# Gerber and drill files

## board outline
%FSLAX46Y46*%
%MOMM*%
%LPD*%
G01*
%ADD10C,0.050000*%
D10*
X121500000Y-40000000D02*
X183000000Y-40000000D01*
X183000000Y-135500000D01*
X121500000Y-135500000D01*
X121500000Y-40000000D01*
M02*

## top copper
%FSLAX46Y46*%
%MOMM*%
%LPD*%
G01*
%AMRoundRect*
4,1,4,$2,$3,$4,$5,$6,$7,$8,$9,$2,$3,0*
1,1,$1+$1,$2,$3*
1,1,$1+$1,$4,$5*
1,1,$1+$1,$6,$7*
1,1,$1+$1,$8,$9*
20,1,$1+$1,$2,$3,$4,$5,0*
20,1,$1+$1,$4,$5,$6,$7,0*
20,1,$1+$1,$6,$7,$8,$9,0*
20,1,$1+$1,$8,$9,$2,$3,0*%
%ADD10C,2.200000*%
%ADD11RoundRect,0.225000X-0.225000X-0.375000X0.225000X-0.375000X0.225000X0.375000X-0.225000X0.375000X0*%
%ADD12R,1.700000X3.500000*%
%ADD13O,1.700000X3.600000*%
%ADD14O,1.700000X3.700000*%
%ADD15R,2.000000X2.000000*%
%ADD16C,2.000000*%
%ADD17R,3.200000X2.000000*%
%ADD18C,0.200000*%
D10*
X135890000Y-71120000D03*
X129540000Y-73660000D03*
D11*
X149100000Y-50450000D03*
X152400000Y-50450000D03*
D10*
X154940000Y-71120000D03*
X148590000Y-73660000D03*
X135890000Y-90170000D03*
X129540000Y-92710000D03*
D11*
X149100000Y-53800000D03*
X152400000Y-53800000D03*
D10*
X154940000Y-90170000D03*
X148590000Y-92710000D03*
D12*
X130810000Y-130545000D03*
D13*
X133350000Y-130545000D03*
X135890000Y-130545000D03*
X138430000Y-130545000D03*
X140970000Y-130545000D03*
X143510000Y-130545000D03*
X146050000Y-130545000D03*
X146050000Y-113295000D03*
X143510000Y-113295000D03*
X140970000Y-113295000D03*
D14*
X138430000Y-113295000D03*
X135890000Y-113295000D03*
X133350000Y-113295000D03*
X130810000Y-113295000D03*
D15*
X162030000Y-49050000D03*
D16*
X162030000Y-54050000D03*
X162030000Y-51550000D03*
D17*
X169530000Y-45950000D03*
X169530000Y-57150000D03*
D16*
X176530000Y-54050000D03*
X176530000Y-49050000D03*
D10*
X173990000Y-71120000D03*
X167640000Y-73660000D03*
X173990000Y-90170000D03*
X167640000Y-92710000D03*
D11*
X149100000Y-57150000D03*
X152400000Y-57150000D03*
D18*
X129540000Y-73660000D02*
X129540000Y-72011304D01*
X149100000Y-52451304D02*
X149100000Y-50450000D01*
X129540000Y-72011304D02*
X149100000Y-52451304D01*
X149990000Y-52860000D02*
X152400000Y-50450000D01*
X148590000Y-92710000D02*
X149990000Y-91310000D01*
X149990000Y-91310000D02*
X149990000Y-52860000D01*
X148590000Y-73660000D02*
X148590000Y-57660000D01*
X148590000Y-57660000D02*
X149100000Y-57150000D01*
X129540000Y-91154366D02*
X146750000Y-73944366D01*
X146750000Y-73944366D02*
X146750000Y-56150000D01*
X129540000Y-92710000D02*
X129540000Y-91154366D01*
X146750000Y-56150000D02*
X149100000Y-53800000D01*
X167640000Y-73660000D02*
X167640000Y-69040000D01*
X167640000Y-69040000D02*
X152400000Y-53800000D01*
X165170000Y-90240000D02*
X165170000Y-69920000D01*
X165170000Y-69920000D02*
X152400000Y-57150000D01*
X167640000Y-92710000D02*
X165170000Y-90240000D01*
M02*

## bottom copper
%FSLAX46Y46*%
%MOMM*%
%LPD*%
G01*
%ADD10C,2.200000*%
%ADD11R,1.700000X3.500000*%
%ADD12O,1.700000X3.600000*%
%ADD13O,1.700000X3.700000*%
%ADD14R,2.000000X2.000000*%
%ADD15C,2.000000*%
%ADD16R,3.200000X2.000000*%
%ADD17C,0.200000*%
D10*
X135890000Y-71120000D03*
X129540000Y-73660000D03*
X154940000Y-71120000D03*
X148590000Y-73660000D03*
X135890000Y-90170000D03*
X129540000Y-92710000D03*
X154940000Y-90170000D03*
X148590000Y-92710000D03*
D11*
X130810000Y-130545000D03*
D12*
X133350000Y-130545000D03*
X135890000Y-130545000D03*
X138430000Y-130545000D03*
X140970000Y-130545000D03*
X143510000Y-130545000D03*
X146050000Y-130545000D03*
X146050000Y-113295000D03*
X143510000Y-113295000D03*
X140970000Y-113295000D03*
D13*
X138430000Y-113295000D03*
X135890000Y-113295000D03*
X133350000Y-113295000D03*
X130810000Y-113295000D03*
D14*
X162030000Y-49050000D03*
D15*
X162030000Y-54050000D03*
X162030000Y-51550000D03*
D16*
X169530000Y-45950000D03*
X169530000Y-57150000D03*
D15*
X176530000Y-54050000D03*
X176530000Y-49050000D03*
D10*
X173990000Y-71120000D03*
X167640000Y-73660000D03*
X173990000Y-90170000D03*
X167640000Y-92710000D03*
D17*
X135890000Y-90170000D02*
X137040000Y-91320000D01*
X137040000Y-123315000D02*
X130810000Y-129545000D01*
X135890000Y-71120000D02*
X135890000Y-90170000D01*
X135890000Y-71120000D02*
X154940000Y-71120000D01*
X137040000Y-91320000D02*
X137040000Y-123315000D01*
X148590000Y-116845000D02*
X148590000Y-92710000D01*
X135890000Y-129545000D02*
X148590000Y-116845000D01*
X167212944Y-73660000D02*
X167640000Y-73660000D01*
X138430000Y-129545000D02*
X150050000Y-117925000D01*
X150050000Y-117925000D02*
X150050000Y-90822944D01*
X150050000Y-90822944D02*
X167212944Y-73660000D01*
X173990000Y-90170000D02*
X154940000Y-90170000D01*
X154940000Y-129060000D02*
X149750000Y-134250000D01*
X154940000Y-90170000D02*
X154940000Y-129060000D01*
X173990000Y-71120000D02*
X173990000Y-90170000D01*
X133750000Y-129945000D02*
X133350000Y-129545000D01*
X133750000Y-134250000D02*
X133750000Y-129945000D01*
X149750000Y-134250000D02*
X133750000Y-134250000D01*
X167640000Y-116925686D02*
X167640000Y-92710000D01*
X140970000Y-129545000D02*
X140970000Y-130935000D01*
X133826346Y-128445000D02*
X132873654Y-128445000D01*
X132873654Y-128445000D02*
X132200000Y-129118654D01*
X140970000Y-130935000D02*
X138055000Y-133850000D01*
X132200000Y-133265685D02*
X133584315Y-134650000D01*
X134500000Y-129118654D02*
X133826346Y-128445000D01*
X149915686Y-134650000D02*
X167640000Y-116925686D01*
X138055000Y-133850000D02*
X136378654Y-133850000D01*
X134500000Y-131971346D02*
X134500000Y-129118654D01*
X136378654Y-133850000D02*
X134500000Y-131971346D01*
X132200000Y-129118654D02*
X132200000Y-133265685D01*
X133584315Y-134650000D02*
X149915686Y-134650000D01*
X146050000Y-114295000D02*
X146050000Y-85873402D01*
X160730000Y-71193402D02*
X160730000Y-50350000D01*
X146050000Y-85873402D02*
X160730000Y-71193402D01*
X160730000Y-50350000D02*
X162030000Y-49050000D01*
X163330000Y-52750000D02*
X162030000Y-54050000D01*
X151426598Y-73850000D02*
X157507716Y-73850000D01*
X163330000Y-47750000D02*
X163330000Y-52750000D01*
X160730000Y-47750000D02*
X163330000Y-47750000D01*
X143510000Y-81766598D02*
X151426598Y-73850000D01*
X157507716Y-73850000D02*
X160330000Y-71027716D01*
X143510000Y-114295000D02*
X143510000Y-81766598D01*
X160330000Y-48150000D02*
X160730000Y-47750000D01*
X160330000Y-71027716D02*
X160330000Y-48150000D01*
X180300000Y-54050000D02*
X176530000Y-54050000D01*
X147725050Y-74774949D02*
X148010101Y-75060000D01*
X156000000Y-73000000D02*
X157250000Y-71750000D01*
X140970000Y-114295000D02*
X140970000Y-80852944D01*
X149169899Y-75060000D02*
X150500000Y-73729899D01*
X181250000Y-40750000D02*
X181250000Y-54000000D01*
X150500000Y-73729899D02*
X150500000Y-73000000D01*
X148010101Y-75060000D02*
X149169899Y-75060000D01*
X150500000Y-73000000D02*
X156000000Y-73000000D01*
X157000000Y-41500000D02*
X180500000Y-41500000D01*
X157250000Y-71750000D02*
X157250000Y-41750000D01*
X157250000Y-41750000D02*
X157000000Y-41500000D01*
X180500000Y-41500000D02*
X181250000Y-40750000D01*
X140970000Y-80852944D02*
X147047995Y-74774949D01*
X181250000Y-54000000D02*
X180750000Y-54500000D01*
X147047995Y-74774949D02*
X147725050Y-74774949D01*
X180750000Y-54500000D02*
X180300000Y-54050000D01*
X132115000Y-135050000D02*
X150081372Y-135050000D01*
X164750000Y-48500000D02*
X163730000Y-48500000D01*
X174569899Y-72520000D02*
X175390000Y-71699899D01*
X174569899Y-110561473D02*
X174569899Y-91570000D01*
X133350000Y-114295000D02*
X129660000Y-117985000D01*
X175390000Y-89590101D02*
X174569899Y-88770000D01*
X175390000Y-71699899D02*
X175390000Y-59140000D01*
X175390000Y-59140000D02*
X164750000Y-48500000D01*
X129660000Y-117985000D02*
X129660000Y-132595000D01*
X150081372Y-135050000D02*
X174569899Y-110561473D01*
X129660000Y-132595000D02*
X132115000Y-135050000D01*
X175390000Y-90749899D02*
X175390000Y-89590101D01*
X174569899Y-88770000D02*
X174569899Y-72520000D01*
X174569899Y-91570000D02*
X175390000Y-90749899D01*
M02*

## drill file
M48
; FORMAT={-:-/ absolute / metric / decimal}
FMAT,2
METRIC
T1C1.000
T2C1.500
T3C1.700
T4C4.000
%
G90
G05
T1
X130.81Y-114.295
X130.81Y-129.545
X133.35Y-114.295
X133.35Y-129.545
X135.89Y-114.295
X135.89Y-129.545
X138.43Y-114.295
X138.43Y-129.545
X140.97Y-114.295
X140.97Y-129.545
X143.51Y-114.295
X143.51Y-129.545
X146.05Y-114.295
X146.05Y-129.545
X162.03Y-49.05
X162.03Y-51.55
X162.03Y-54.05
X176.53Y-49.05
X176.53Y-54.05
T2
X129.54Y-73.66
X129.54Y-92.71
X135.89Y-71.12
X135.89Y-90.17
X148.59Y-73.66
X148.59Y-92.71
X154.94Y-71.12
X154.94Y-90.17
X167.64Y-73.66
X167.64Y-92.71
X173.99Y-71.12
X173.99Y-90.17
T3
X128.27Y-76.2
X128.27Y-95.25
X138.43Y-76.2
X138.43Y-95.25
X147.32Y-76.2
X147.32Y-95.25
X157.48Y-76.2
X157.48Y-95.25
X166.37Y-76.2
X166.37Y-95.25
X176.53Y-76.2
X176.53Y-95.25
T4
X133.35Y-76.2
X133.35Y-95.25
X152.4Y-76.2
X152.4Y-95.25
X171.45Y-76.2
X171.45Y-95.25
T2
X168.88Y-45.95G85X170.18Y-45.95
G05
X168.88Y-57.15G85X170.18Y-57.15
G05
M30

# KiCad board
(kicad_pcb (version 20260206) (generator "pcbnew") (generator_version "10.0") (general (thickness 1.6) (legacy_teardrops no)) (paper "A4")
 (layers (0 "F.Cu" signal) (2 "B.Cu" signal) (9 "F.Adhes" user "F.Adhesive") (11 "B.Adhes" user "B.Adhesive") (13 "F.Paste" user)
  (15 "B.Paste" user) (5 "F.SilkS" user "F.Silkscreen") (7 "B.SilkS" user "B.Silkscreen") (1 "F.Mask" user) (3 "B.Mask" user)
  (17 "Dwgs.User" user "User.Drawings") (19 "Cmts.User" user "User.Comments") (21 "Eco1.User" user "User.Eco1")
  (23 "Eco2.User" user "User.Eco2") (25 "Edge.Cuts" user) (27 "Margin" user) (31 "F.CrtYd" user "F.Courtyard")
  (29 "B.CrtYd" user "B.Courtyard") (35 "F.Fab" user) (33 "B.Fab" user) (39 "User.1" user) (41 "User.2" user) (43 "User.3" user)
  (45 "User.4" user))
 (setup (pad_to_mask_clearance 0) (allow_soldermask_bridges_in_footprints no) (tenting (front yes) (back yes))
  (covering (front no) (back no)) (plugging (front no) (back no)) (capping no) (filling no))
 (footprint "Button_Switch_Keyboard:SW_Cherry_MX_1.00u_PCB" (layer "F.Cu") (at 135.89 71.12)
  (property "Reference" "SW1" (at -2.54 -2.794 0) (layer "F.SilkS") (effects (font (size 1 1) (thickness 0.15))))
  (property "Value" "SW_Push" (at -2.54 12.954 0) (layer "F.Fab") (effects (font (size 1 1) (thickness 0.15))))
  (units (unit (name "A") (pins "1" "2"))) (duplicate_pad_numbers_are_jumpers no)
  (pad "" np_thru_hole circle (at -7.62 5.08) (size 1.7 1.7) (drill 1.7) (layers "*.Cu" "*.Mask"))
  (pad "" np_thru_hole circle (at -2.54 5.08) (size 4 4) (drill 4) (layers "*.Cu" "*.Mask"))
  (pad "" np_thru_hole circle (at 2.54 5.08) (size 1.7 1.7) (drill 1.7) (layers "*.Cu" "*.Mask"))
  (pad "1" thru_hole circle (at 0 0) (size 2.2 2.2) (drill 1.5) (layers "*.Cu" "*.Mask") (remove_unused_layers no)
   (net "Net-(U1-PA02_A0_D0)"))
  (pad "2" thru_hole circle (at -6.35 2.54) (size 2.2 2.2) (drill 1.5) (layers "*.Cu" "*.Mask") (remove_unused_layers no) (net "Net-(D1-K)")))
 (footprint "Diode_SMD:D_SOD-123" (layer "F.Cu") (at 150.75 50.45)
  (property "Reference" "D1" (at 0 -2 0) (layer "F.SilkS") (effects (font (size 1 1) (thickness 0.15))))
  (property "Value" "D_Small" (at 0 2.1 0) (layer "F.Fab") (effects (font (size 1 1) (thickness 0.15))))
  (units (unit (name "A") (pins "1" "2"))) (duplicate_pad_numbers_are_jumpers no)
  (pad "1" smd roundrect (at -1.65 0) (size 0.9 1.2) (layers "F.Cu" "F.Mask" "F.Paste") (roundrect_rratio 0.25) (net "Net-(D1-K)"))
  (pad "2" smd roundrect (at 1.65 0) (size 0.9 1.2) (layers "F.Cu" "F.Mask" "F.Paste") (roundrect_rratio 0.25) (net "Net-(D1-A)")))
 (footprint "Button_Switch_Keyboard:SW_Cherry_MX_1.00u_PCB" (layer "F.Cu") (at 154.94 71.12)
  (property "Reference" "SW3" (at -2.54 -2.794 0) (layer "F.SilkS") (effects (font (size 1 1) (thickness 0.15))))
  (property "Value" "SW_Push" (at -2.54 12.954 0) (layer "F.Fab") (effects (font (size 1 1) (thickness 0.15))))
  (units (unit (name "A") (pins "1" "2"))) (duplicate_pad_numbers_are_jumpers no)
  (pad "" np_thru_hole circle (at -7.62 5.08) (size 1.7 1.7) (drill 1.7) (layers "*.Cu" "*.Mask"))
  (pad "" np_thru_hole circle (at -2.54 5.08) (size 4 4) (drill 4) (layers "*.Cu" "*.Mask"))
  (pad "" np_thru_hole circle (at 2.54 5.08) (size 1.7 1.7) (drill 1.7) (layers "*.Cu" "*.Mask"))
  (pad "1" thru_hole circle (at 0 0) (size 2.2 2.2) (drill 1.5) (layers "*.Cu" "*.Mask") (remove_unused_layers no)
   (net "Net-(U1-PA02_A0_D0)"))
  (pad "2" thru_hole circle (at -6.35 2.54) (size 2.2 2.2) (drill 1.5) (layers "*.Cu" "*.Mask") (remove_unused_layers no) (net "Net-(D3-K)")))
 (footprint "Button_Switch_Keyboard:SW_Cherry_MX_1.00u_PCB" (layer "F.Cu") (at 135.89 90.17)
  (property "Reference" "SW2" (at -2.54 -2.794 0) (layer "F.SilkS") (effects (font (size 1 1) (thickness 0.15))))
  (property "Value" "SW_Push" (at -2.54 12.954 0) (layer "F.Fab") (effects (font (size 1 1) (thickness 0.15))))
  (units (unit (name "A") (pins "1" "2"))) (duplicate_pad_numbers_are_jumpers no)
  (pad "" np_thru_hole circle (at -7.62 5.08) (size 1.7 1.7) (drill 1.7) (layers "*.Cu" "*.Mask"))
  (pad "" np_thru_hole circle (at -2.54 5.08) (size 4 4) (drill 4) (layers "*.Cu" "*.Mask"))
  (pad "" np_thru_hole circle (at 2.54 5.08) (size 1.7 1.7) (drill 1.7) (layers "*.Cu" "*.Mask"))
  (pad "1" thru_hole circle (at 0 0) (size 2.2 2.2) (drill 1.5) (layers "*.Cu" "*.Mask") (remove_unused_layers no)
   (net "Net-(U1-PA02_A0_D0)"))
  (pad "2" thru_hole circle (at -6.35 2.54) (size 2.2 2.2) (drill 1.5) (layers "*.Cu" "*.Mask") (remove_unused_layers no) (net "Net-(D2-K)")))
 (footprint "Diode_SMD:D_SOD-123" (layer "F.Cu") (at 150.75 53.8)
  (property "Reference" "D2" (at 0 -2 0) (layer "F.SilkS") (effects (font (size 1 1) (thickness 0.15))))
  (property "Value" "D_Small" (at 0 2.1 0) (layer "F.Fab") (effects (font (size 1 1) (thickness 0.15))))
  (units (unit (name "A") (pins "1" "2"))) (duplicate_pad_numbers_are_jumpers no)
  (pad "1" smd roundrect (at -1.65 0) (size 0.9 1.2) (layers "F.Cu" "F.Mask" "F.Paste") (roundrect_rratio 0.25) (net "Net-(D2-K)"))
  (pad "2" smd roundrect (at 1.65 0) (size 0.9 1.2) (layers "F.Cu" "F.Mask" "F.Paste") (roundrect_rratio 0.25) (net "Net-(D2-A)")))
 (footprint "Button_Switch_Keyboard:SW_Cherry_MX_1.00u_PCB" (layer "F.Cu") (at 154.94 90.17)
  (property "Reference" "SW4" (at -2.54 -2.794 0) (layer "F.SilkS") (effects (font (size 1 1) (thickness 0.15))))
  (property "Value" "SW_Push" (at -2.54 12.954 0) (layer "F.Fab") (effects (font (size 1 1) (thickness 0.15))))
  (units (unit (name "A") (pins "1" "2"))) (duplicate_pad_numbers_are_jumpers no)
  (pad "" np_thru_hole circle (at -7.62 5.08) (size 1.7 1.7) (drill 1.7) (layers "*.Cu" "*.Mask"))
  (pad "" np_thru_hole circle (at -2.54 5.08) (size 4 4) (drill 4) (layers "*.Cu" "*.Mask"))
  (pad "" np_thru_hole circle (at 2.54 5.08) (size 1.7 1.7) (drill 1.7) (layers "*.Cu" "*.Mask"))
  (pad "1" thru_hole circle (at 0 0) (size 2.2 2.2) (drill 1.5) (layers "*.Cu" "*.Mask") (remove_unused_layers no)
   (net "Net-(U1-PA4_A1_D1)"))
  (pad "2" thru_hole circle (at -6.35 2.54) (size 2.2 2.2) (drill 1.5) (layers "*.Cu" "*.Mask") (remove_unused_layers no) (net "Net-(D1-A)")))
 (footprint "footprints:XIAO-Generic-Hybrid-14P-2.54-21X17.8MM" (layer "F.Cu") (at 138.43 121.92 90)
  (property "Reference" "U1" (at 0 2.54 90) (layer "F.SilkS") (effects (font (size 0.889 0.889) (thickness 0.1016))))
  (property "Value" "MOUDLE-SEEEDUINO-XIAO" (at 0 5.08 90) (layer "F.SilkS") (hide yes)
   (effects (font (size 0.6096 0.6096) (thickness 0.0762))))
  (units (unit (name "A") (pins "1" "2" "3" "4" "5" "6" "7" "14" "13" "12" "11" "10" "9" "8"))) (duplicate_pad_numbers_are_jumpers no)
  (pad "1" thru_hole rect (at -7.625 -7.62 90) (size 3.5 1.7) (drill 1 (offset -1 0)) (layers "*.Cu" "*.Mask") (remove_unused_layers no)
   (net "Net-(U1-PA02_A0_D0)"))
  (pad "2" thru_hole oval (at -7.625 -5.08 90) (size 3.6 1.7) (drill 1 (offset -1 0)) (layers "*.Cu" "*.Mask") (remove_unused_layers no)
   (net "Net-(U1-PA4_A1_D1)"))
  (pad "3" thru_hole oval (at -7.625 -2.54 90) (size 3.6 1.7) (drill 1 (offset -1 0)) (layers "*.Cu" "*.Mask") (remove_unused_layers no)
   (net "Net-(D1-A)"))
  (pad "4" thru_hole oval (at -7.625 0 90) (size 3.6 1.7) (drill 1 (offset -1 0)) (layers "*.Cu" "*.Mask") (remove_unused_layers no)
   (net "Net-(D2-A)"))
  (pad "5" thru_hole oval (at -7.625 2.54 90) (size 3.6 1.7) (drill 1 (offset -1 0)) (layers "*.Cu" "*.Mask") (remove_unused_layers no)
   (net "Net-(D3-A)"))
  (pad "6" thru_hole oval (at -7.625 5.08 270) (size 3.6 1.7) (drill 1 (offset 1 0)) (layers "*.Cu" "*.Mask") (remove_unused_layers no)
   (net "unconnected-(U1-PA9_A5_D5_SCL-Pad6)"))
  (pad "7" thru_hole oval (at -7.625 7.62 90) (size 3.6 1.7) (drill 1 (offset -1 0)) (layers "*.Cu" "*.Mask") (remove_unused_layers no)
   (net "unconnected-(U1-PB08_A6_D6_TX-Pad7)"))
  (pad "8" thru_hole oval (at 7.625 7.62 90) (size 3.6 1.7) (drill 1 (offset 1 0)) (layers "*.Cu" "*.Mask") (remove_unused_layers no)
   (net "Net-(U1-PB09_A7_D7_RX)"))
  (pad "9" thru_hole oval (at 7.625 5.08 90) (size 3.6 1.7) (drill 1 (offset 1 0)) (layers "*.Cu" "*.Mask") (remove_unused_layers no)
   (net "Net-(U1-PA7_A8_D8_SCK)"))
  (pad "10" thru_hole oval (at 7.625 2.54 90) (size 3.6 1.7) (drill 1 (offset 1 0)) (layers "*.Cu" "*.Mask") (remove_unused_layers no)
   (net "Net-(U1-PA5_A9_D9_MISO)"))
  (pad "11" thru_hole oval (at 7.625 0 90) (size 3.7 1.7) (drill 1 (offset 1 0)) (layers "*.Cu" "*.Mask") (remove_unused_layers no)
   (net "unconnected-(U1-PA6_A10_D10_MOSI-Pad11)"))
  (pad "12" thru_hole oval (at 7.625 -2.54 90) (size 3.7 1.7) (drill 1 (offset 1 0)) (layers "*.Cu" "*.Mask") (remove_unused_layers no)
   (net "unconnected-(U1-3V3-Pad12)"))
  (pad "13" thru_hole oval (at 7.625 -5.08 90) (size 3.7 1.7) (drill 1 (offset 1 0)) (layers "*.Cu" "*.Mask") (remove_unused_layers no)
   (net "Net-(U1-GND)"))
  (pad "14" thru_hole oval (at 7.625 -7.62 90) (size 3.7 1.7) (drill 1 (offset 1 0)) (layers "*.Cu" "*.Mask") (remove_unused_layers no)
   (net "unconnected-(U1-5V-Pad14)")))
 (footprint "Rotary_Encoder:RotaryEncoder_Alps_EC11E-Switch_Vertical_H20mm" (layer "F.Cu") (at 162.03 49.05)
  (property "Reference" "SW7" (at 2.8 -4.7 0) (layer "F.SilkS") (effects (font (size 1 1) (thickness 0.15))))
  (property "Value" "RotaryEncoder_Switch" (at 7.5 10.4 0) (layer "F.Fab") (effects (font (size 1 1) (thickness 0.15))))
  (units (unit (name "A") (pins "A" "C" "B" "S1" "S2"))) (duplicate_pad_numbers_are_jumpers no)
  (pad "A" thru_hole rect (at 0 0) (size 2 2) (drill 1) (layers "*.Cu" "*.Mask") (remove_unused_layers no) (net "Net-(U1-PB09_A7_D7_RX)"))
  (pad "B" thru_hole circle (at 0 5) (size 2 2) (drill 1) (layers "*.Cu" "*.Mask") (remove_unused_layers no) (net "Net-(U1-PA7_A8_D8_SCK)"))
  (pad "C" thru_hole circle (at 0 2.5) (size 2 2) (drill 1) (layers "*.Cu" "*.Mask") (remove_unused_layers no) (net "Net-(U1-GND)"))
  (pad "MP" thru_hole rect (at 7.5 -3.1) (size 3.2 2) (drill oval 2.8 1.5) (layers "*.Cu" "*.Mask") (remove_unused_layers no))
  (pad "MP" thru_hole rect (at 7.5 8.1) (size 3.2 2) (drill oval 2.8 1.5) (layers "*.Cu" "*.Mask") (remove_unused_layers no))
  (pad "S1" thru_hole circle (at 14.5 5) (size 2 2) (drill 1) (layers "*.Cu" "*.Mask") (remove_unused_layers no)
   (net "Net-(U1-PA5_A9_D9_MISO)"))
  (pad "S2" thru_hole circle (at 14.5 0) (size 2 2) (drill 1) (layers "*.Cu" "*.Mask") (remove_unused_layers no) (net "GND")))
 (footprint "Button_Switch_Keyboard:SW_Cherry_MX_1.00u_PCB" (layer "F.Cu") (at 173.99 71.12)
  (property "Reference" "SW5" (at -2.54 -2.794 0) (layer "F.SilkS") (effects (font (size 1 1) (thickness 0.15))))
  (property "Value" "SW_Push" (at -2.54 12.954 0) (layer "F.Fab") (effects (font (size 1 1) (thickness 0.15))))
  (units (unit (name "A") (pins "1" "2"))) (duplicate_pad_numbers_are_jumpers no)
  (pad "" np_thru_hole circle (at -7.62 5.08) (size 1.7 1.7) (drill 1.7) (layers "*.Cu" "*.Mask"))
  (pad "" np_thru_hole circle (at -2.54 5.08) (size 4 4) (drill 4) (layers "*.Cu" "*.Mask"))
  (pad "" np_thru_hole circle (at 2.54 5.08) (size 1.7 1.7) (drill 1.7) (layers "*.Cu" "*.Mask"))
  (pad "1" thru_hole circle (at 0 0) (size 2.2 2.2) (drill 1.5) (layers "*.Cu" "*.Mask") (remove_unused_layers no)
   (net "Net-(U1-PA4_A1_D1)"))
  (pad "2" thru_hole circle (at -6.35 2.54) (size 2.2 2.2) (drill 1.5) (layers "*.Cu" "*.Mask") (remove_unused_layers no) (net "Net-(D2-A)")))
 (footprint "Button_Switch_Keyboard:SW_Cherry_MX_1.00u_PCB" (layer "F.Cu") (at 173.99 90.17)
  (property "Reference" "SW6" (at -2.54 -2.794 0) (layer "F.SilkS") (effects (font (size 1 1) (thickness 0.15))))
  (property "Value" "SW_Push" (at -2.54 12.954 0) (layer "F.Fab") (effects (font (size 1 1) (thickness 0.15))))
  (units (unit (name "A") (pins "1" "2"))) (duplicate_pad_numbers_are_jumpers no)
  (pad "" np_thru_hole circle (at -7.62 5.08) (size 1.7 1.7) (drill 1.7) (layers "*.Cu" "*.Mask"))
  (pad "" np_thru_hole circle (at -2.54 5.08) (size 4 4) (drill 4) (layers "*.Cu" "*.Mask"))
  (pad "" np_thru_hole circle (at 2.54 5.08) (size 1.7 1.7) (drill 1.7) (layers "*.Cu" "*.Mask"))
  (pad "1" thru_hole circle (at 0 0) (size 2.2 2.2) (drill 1.5) (layers "*.Cu" "*.Mask") (remove_unused_layers no)
   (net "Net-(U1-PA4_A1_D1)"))
  (pad "2" thru_hole circle (at -6.35 2.54) (size 2.2 2.2) (drill 1.5) (layers "*.Cu" "*.Mask") (remove_unused_layers no) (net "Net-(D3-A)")))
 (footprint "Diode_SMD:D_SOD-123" (layer "F.Cu") (at 150.75 57.15)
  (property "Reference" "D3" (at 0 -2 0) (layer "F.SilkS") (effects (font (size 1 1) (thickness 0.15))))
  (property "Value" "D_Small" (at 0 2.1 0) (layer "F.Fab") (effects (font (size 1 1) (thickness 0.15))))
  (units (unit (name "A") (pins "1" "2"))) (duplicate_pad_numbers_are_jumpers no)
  (pad "1" smd roundrect (at -1.65 0) (size 0.9 1.2) (layers "F.Cu" "F.Mask" "F.Paste") (roundrect_rratio 0.25) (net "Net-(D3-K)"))
  (pad "2" smd roundrect (at 1.65 0) (size 0.9 1.2) (layers "F.Cu" "F.Mask" "F.Paste") (roundrect_rratio 0.25) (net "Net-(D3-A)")))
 (gr_rect (start 121.5 40) (end 183 135.5) (stroke (width 0.05) (type default)) (fill no) (layer "Edge.Cuts"))
 (segment (start 135.89 90.17) (end 137.04 91.32) (width 0.2) (layer "B.Cu") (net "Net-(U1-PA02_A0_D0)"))
 (segment (start 137.04 123.315) (end 130.81 129.545) (width 0.2) (layer "B.Cu") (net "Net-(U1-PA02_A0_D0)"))
 (segment (start 135.89 71.12) (end 135.89 90.17) (width 0.2) (layer "B.Cu") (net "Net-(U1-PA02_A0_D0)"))
 (segment (start 135.89 71.12) (end 154.94 71.12) (width 0.2) (layer "B.Cu") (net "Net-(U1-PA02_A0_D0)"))
 (segment (start 137.04 91.32) (end 137.04 123.315) (width 0.2) (layer "B.Cu") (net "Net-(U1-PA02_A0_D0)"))
 (segment (start 129.54 73.66) (end 129.54 72.011304) (width 0.2) (layer "F.Cu") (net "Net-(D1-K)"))
 (segment (start 149.1 52.451304) (end 149.1 50.45) (width 0.2) (layer "F.Cu") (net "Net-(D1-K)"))
 (segment (start 129.54 72.011304) (end 149.1 52.451304) (width 0.2) (layer "F.Cu") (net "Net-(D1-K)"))
 (segment (start 149.99 52.86) (end 152.4 50.45) (width 0.2) (layer "F.Cu") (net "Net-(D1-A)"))
 (segment (start 148.59 92.71) (end 149.99 91.31) (width 0.2) (layer "F.Cu") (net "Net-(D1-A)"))
 (segment (start 149.99 91.31) (end 149.99 52.86) (width 0.2) (layer "F.Cu") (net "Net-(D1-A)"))
 (segment (start 148.59 116.845) (end 148.59 92.71) (width 0.2) (layer "B.Cu") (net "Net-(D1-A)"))
 (segment (start 135.89 129.545) (end 148.59 116.845) (width 0.2) (layer "B.Cu") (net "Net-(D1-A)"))
 (segment (start 148.59 73.66) (end 148.59 57.66) (width 0.2) (layer "F.Cu") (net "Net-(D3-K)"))
 (segment (start 148.59 57.66) (end 149.1 57.15) (width 0.2) (layer "F.Cu") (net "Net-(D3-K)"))
 (segment (start 129.54 91.154366) (end 146.75 73.944366) (width 0.2) (layer "F.Cu") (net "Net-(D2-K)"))
 (segment (start 146.75 73.944366) (end 146.75 56.15) (width 0.2) (layer "F.Cu") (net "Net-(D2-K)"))
 (segment (start 129.54 92.71) (end 129.54 91.154366) (width 0.2) (layer "F.Cu") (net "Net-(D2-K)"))
 (segment (start 146.75 56.15) (end 149.1 53.8) (width 0.2) (layer "F.Cu") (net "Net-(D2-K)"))
 (segment (start 167.64 73.66) (end 167.64 69.04) (width 0.2) (layer "F.Cu") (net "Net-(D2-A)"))
 (segment (start 167.64 69.04) (end 152.4 53.8) (width 0.2) (layer "F.Cu") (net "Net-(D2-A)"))
 (segment (start 167.212944 73.66) (end 167.64 73.66) (width 0.2) (layer "B.Cu") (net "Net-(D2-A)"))
 (segment (start 138.43 129.545) (end 150.05 117.925) (width 0.2) (layer "B.Cu") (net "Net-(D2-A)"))
 (segment (start 150.05 117.925) (end 150.05 90.822944) (width 0.2) (layer "B.Cu") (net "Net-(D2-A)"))
 (segment (start 150.05 90.822944) (end 167.212944 73.66) (width 0.2) (layer "B.Cu") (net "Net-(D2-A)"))
 (segment (start 173.99 90.17) (end 154.94 90.17) (width 0.2) (layer "B.Cu") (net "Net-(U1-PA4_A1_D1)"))
 (segment (start 154.94 129.06) (end 149.75 134.25) (width 0.2) (layer "B.Cu") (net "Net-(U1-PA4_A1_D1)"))
 (segment (start 154.94 90.17) (end 154.94 129.06) (width 0.2) (layer "B.Cu") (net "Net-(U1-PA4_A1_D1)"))
 (segment (start 173.99 71.12) (end 173.99 90.17) (width 0.2) (layer "B.Cu") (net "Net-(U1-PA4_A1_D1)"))
 (segment (start 133.75 129.945) (end 133.35 129.545) (width 0.2) (layer "B.Cu") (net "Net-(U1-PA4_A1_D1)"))
 (segment (start 133.75 134.25) (end 133.75 129.945) (width 0.2) (layer "B.Cu") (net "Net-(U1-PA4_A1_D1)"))
 (segment (start 149.75 134.25) (end 133.75 134.25) (width 0.2) (layer "B.Cu") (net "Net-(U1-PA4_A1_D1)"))
 (segment (start 165.17 90.24) (end 165.17 69.92) (width 0.2) (layer "F.Cu") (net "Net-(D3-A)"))
 (segment (start 165.17 69.92) (end 152.4 57.15) (width 0.2) (layer "F.Cu") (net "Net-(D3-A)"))
 (segment (start 167.64 92.71) (end 165.17 90.24) (width 0.2) (layer "F.Cu") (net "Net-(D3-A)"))
 (segment (start 167.64 116.925686) (end 167.64 92.71) (width 0.2) (layer "B.Cu") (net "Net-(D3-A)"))
 (segment (start 140.97 129.545) (end 140.97 130.935) (width 0.2) (layer "B.Cu") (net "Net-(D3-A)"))
 (segment (start 133.826346 128.445) (end 132.873654 128.445) (width 0.2) (layer "B.Cu") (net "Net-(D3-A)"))
 (segment (start 132.873654 128.445) (end 132.2 129.118654) (width 0.2) (layer "B.Cu") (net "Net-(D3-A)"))
 (segment (start 140.97 130.935) (end 138.055 133.85) (width 0.2) (layer "B.Cu") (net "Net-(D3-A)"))
 (segment (start 132.2 133.265685) (end 133.584315 134.65) (width 0.2) (layer "B.Cu") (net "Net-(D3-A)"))
 (segment (start 134.5 129.118654) (end 133.826346 128.445) (width 0.2) (layer "B.Cu") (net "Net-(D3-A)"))
 (segment (start 149.915686 134.65) (end 167.64 116.925686) (width 0.2) (layer "B.Cu") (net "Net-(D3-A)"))
 (segment (start 138.055 133.85) (end 136.378654 133.85) (width 0.2) (layer "B.Cu") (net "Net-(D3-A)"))
 (segment (start 134.5 131.971346) (end 134.5 129.118654) (width 0.2) (layer "B.Cu") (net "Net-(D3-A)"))
 (segment (start 136.378654 133.85) (end 134.5 131.971346) (width 0.2) (layer "B.Cu") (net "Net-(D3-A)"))
 (segment (start 132.2 129.118654) (end 132.2 133.265685) (width 0.2) (layer "B.Cu") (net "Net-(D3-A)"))
 (segment (start 133.584315 134.65) (end 149.915686 134.65) (width 0.2) (layer "B.Cu") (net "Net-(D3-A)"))
 (segment (start 146.05 114.295) (end 146.05 85.873402) (width 0.2) (layer "B.Cu") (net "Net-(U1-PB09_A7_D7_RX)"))
 (segment (start 160.73 71.193402) (end 160.73 50.35) (width 0.2) (layer "B.Cu") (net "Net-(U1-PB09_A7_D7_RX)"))
 (segment (start 146.05 85.873402) (end 160.73 71.193402) (width 0.2) (layer "B.Cu") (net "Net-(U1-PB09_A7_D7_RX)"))
 (segment (start 160.73 50.35) (end 162.03 49.05) (width 0.2) (layer "B.Cu") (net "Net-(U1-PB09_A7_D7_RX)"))
 (segment (start 163.33 52.75) (end 162.03 54.05) (width 0.2) (layer "B.Cu") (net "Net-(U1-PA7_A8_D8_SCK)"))
 (segment (start 151.426598 73.85) (end 157.507716 73.85) (width 0.2) (layer "B.Cu") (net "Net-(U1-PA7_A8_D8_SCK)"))
 (segment (start 163.33 47.75) (end 163.33 52.75) (width 0.2) (layer "B.Cu") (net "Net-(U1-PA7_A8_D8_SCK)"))
 (segment (start 160.73 47.75) (end 163.33 47.75) (width 0.2) (layer "B.Cu") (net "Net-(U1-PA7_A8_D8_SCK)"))
 (segment (start 143.51 81.766598) (end 151.426598 73.85) (width 0.2) (layer "B.Cu") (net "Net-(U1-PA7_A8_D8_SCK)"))
 (segment (start 157.507716 73.85) (end 160.33 71.027716) (width 0.2) (layer "B.Cu") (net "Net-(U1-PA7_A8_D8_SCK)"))
 (segment (start 143.51 114.295) (end 143.51 81.766598) (width 0.2) (layer "B.Cu") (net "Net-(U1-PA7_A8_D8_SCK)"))
 (segment (start 160.33 48.15) (end 160.73 47.75) (width 0.2) (layer "B.Cu") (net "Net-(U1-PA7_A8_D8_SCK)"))
 (segment (start 160.33 71.027716) (end 160.33 48.15) (width 0.2) (layer "B.Cu") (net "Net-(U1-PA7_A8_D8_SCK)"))
 (segment (start 180.3 54.05) (end 176.53 54.05) (width 0.2) (layer "B.Cu") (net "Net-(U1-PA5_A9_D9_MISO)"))
 (segment (start 147.72505 74.774949) (end 148.010101 75.06) (width 0.2) (layer "B.Cu") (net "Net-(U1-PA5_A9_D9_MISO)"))
 (segment (start 156 73) (end 157.25 71.75) (width 0.2) (layer "B.Cu") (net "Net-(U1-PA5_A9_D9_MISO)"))
 (segment (start 140.97 114.295) (end 140.97 80.852944) (width 0.2) (layer "B.Cu") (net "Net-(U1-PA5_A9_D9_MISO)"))
 (segment (start 149.169899 75.06) (end 150.5 73.729899) (width 0.2) (layer "B.Cu") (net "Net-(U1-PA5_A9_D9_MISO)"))
 (segment (start 181.25 40.75) (end 181.25 54) (width 0.2) (layer "B.Cu") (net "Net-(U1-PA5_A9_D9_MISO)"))
 (segment (start 150.5 73.729899) (end 150.5 73) (width 0.2) (layer "B.Cu") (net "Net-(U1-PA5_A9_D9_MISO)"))
 (segment (start 148.010101 75.06) (end 149.169899 75.06) (width 0.2) (layer "B.Cu") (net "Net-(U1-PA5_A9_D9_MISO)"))
 (segment (start 150.5 73) (end 156 73) (width 0.2) (layer "B.Cu") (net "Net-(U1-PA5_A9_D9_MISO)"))
 (segment (start 157 41.5) (end 180.5 41.5) (width 0.2) (layer "B.Cu") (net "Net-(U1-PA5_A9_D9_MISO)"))
 (segment (start 157.25 71.75) (end 157.25 41.75) (width 0.2) (layer "B.Cu") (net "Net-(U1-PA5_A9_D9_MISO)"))
 (segment (start 157.25 41.75) (end 157 41.5) (width 0.2) (layer "B.Cu") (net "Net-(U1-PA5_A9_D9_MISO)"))
 (segment (start 180.5 41.5) (end 181.25 40.75) (width 0.2) (layer "B.Cu") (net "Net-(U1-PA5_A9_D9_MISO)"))
 (segment (start 140.97 80.852944) (end 147.047995 74.774949) (width 0.2) (layer "B.Cu") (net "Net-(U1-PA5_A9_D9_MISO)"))
 (segment (start 181.25 54) (end 180.75 54.5) (width 0.2) (layer "B.Cu") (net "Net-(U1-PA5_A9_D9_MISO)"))
 (segment (start 147.047995 74.774949) (end 147.72505 74.774949) (width 0.2) (layer "B.Cu") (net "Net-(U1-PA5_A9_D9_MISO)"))
 (segment (start 180.75 54.5) (end 180.3 54.05) (width 0.2) (layer "B.Cu") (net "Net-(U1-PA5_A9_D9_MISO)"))
 (segment (start 132.115 135.05) (end 150.081372 135.05) (width 0.2) (layer "B.Cu") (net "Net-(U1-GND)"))
 (segment (start 164.75 48.5) (end 163.73 48.5) (width 0.2) (layer "B.Cu") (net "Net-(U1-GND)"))
 (segment (start 174.569899 72.52) (end 175.39 71.699899) (width 0.2) (layer "B.Cu") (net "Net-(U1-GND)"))
 (segment (start 174.569899 110.561473) (end 174.569899 91.57) (width 0.2) (layer "B.Cu") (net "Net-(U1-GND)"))
 (segment (start 133.35 114.295) (end 129.66 117.985) (width 0.2) (layer "B.Cu") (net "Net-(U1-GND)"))
 (segment (start 175.39 89.590101) (end 174.569899 88.77) (width 0.2) (layer "B.Cu") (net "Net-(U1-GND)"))
 (segment (start 175.39 71.699899) (end 175.39 59.14) (width 0.2) (layer "B.Cu") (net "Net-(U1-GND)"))
 (segment (start 175.39 59.14) (end 164.75 48.5) (width 0.2) (layer "B.Cu") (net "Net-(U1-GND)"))
 (segment (start 129.66 117.985) (end 129.66 132.595) (width 0.2) (layer "B.Cu") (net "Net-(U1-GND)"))
 (segment (start 150.081372 135.05) (end 174.569899 110.561473) (width 0.2) (layer "B.Cu") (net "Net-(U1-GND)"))
 (segment (start 129.66 132.595) (end 132.115 135.05) (width 0.2) (layer "B.Cu") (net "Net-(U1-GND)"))
 (segment (start 175.39 90.749899) (end 175.39 89.590101) (width 0.2) (layer "B.Cu") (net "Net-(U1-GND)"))
 (segment (start 174.569899 88.77) (end 174.569899 72.52) (width 0.2) (layer "B.Cu") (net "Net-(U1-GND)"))
 (segment (start 174.569899 91.57) (end 175.39 90.749899) (width 0.2) (layer "B.Cu") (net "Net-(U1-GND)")))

